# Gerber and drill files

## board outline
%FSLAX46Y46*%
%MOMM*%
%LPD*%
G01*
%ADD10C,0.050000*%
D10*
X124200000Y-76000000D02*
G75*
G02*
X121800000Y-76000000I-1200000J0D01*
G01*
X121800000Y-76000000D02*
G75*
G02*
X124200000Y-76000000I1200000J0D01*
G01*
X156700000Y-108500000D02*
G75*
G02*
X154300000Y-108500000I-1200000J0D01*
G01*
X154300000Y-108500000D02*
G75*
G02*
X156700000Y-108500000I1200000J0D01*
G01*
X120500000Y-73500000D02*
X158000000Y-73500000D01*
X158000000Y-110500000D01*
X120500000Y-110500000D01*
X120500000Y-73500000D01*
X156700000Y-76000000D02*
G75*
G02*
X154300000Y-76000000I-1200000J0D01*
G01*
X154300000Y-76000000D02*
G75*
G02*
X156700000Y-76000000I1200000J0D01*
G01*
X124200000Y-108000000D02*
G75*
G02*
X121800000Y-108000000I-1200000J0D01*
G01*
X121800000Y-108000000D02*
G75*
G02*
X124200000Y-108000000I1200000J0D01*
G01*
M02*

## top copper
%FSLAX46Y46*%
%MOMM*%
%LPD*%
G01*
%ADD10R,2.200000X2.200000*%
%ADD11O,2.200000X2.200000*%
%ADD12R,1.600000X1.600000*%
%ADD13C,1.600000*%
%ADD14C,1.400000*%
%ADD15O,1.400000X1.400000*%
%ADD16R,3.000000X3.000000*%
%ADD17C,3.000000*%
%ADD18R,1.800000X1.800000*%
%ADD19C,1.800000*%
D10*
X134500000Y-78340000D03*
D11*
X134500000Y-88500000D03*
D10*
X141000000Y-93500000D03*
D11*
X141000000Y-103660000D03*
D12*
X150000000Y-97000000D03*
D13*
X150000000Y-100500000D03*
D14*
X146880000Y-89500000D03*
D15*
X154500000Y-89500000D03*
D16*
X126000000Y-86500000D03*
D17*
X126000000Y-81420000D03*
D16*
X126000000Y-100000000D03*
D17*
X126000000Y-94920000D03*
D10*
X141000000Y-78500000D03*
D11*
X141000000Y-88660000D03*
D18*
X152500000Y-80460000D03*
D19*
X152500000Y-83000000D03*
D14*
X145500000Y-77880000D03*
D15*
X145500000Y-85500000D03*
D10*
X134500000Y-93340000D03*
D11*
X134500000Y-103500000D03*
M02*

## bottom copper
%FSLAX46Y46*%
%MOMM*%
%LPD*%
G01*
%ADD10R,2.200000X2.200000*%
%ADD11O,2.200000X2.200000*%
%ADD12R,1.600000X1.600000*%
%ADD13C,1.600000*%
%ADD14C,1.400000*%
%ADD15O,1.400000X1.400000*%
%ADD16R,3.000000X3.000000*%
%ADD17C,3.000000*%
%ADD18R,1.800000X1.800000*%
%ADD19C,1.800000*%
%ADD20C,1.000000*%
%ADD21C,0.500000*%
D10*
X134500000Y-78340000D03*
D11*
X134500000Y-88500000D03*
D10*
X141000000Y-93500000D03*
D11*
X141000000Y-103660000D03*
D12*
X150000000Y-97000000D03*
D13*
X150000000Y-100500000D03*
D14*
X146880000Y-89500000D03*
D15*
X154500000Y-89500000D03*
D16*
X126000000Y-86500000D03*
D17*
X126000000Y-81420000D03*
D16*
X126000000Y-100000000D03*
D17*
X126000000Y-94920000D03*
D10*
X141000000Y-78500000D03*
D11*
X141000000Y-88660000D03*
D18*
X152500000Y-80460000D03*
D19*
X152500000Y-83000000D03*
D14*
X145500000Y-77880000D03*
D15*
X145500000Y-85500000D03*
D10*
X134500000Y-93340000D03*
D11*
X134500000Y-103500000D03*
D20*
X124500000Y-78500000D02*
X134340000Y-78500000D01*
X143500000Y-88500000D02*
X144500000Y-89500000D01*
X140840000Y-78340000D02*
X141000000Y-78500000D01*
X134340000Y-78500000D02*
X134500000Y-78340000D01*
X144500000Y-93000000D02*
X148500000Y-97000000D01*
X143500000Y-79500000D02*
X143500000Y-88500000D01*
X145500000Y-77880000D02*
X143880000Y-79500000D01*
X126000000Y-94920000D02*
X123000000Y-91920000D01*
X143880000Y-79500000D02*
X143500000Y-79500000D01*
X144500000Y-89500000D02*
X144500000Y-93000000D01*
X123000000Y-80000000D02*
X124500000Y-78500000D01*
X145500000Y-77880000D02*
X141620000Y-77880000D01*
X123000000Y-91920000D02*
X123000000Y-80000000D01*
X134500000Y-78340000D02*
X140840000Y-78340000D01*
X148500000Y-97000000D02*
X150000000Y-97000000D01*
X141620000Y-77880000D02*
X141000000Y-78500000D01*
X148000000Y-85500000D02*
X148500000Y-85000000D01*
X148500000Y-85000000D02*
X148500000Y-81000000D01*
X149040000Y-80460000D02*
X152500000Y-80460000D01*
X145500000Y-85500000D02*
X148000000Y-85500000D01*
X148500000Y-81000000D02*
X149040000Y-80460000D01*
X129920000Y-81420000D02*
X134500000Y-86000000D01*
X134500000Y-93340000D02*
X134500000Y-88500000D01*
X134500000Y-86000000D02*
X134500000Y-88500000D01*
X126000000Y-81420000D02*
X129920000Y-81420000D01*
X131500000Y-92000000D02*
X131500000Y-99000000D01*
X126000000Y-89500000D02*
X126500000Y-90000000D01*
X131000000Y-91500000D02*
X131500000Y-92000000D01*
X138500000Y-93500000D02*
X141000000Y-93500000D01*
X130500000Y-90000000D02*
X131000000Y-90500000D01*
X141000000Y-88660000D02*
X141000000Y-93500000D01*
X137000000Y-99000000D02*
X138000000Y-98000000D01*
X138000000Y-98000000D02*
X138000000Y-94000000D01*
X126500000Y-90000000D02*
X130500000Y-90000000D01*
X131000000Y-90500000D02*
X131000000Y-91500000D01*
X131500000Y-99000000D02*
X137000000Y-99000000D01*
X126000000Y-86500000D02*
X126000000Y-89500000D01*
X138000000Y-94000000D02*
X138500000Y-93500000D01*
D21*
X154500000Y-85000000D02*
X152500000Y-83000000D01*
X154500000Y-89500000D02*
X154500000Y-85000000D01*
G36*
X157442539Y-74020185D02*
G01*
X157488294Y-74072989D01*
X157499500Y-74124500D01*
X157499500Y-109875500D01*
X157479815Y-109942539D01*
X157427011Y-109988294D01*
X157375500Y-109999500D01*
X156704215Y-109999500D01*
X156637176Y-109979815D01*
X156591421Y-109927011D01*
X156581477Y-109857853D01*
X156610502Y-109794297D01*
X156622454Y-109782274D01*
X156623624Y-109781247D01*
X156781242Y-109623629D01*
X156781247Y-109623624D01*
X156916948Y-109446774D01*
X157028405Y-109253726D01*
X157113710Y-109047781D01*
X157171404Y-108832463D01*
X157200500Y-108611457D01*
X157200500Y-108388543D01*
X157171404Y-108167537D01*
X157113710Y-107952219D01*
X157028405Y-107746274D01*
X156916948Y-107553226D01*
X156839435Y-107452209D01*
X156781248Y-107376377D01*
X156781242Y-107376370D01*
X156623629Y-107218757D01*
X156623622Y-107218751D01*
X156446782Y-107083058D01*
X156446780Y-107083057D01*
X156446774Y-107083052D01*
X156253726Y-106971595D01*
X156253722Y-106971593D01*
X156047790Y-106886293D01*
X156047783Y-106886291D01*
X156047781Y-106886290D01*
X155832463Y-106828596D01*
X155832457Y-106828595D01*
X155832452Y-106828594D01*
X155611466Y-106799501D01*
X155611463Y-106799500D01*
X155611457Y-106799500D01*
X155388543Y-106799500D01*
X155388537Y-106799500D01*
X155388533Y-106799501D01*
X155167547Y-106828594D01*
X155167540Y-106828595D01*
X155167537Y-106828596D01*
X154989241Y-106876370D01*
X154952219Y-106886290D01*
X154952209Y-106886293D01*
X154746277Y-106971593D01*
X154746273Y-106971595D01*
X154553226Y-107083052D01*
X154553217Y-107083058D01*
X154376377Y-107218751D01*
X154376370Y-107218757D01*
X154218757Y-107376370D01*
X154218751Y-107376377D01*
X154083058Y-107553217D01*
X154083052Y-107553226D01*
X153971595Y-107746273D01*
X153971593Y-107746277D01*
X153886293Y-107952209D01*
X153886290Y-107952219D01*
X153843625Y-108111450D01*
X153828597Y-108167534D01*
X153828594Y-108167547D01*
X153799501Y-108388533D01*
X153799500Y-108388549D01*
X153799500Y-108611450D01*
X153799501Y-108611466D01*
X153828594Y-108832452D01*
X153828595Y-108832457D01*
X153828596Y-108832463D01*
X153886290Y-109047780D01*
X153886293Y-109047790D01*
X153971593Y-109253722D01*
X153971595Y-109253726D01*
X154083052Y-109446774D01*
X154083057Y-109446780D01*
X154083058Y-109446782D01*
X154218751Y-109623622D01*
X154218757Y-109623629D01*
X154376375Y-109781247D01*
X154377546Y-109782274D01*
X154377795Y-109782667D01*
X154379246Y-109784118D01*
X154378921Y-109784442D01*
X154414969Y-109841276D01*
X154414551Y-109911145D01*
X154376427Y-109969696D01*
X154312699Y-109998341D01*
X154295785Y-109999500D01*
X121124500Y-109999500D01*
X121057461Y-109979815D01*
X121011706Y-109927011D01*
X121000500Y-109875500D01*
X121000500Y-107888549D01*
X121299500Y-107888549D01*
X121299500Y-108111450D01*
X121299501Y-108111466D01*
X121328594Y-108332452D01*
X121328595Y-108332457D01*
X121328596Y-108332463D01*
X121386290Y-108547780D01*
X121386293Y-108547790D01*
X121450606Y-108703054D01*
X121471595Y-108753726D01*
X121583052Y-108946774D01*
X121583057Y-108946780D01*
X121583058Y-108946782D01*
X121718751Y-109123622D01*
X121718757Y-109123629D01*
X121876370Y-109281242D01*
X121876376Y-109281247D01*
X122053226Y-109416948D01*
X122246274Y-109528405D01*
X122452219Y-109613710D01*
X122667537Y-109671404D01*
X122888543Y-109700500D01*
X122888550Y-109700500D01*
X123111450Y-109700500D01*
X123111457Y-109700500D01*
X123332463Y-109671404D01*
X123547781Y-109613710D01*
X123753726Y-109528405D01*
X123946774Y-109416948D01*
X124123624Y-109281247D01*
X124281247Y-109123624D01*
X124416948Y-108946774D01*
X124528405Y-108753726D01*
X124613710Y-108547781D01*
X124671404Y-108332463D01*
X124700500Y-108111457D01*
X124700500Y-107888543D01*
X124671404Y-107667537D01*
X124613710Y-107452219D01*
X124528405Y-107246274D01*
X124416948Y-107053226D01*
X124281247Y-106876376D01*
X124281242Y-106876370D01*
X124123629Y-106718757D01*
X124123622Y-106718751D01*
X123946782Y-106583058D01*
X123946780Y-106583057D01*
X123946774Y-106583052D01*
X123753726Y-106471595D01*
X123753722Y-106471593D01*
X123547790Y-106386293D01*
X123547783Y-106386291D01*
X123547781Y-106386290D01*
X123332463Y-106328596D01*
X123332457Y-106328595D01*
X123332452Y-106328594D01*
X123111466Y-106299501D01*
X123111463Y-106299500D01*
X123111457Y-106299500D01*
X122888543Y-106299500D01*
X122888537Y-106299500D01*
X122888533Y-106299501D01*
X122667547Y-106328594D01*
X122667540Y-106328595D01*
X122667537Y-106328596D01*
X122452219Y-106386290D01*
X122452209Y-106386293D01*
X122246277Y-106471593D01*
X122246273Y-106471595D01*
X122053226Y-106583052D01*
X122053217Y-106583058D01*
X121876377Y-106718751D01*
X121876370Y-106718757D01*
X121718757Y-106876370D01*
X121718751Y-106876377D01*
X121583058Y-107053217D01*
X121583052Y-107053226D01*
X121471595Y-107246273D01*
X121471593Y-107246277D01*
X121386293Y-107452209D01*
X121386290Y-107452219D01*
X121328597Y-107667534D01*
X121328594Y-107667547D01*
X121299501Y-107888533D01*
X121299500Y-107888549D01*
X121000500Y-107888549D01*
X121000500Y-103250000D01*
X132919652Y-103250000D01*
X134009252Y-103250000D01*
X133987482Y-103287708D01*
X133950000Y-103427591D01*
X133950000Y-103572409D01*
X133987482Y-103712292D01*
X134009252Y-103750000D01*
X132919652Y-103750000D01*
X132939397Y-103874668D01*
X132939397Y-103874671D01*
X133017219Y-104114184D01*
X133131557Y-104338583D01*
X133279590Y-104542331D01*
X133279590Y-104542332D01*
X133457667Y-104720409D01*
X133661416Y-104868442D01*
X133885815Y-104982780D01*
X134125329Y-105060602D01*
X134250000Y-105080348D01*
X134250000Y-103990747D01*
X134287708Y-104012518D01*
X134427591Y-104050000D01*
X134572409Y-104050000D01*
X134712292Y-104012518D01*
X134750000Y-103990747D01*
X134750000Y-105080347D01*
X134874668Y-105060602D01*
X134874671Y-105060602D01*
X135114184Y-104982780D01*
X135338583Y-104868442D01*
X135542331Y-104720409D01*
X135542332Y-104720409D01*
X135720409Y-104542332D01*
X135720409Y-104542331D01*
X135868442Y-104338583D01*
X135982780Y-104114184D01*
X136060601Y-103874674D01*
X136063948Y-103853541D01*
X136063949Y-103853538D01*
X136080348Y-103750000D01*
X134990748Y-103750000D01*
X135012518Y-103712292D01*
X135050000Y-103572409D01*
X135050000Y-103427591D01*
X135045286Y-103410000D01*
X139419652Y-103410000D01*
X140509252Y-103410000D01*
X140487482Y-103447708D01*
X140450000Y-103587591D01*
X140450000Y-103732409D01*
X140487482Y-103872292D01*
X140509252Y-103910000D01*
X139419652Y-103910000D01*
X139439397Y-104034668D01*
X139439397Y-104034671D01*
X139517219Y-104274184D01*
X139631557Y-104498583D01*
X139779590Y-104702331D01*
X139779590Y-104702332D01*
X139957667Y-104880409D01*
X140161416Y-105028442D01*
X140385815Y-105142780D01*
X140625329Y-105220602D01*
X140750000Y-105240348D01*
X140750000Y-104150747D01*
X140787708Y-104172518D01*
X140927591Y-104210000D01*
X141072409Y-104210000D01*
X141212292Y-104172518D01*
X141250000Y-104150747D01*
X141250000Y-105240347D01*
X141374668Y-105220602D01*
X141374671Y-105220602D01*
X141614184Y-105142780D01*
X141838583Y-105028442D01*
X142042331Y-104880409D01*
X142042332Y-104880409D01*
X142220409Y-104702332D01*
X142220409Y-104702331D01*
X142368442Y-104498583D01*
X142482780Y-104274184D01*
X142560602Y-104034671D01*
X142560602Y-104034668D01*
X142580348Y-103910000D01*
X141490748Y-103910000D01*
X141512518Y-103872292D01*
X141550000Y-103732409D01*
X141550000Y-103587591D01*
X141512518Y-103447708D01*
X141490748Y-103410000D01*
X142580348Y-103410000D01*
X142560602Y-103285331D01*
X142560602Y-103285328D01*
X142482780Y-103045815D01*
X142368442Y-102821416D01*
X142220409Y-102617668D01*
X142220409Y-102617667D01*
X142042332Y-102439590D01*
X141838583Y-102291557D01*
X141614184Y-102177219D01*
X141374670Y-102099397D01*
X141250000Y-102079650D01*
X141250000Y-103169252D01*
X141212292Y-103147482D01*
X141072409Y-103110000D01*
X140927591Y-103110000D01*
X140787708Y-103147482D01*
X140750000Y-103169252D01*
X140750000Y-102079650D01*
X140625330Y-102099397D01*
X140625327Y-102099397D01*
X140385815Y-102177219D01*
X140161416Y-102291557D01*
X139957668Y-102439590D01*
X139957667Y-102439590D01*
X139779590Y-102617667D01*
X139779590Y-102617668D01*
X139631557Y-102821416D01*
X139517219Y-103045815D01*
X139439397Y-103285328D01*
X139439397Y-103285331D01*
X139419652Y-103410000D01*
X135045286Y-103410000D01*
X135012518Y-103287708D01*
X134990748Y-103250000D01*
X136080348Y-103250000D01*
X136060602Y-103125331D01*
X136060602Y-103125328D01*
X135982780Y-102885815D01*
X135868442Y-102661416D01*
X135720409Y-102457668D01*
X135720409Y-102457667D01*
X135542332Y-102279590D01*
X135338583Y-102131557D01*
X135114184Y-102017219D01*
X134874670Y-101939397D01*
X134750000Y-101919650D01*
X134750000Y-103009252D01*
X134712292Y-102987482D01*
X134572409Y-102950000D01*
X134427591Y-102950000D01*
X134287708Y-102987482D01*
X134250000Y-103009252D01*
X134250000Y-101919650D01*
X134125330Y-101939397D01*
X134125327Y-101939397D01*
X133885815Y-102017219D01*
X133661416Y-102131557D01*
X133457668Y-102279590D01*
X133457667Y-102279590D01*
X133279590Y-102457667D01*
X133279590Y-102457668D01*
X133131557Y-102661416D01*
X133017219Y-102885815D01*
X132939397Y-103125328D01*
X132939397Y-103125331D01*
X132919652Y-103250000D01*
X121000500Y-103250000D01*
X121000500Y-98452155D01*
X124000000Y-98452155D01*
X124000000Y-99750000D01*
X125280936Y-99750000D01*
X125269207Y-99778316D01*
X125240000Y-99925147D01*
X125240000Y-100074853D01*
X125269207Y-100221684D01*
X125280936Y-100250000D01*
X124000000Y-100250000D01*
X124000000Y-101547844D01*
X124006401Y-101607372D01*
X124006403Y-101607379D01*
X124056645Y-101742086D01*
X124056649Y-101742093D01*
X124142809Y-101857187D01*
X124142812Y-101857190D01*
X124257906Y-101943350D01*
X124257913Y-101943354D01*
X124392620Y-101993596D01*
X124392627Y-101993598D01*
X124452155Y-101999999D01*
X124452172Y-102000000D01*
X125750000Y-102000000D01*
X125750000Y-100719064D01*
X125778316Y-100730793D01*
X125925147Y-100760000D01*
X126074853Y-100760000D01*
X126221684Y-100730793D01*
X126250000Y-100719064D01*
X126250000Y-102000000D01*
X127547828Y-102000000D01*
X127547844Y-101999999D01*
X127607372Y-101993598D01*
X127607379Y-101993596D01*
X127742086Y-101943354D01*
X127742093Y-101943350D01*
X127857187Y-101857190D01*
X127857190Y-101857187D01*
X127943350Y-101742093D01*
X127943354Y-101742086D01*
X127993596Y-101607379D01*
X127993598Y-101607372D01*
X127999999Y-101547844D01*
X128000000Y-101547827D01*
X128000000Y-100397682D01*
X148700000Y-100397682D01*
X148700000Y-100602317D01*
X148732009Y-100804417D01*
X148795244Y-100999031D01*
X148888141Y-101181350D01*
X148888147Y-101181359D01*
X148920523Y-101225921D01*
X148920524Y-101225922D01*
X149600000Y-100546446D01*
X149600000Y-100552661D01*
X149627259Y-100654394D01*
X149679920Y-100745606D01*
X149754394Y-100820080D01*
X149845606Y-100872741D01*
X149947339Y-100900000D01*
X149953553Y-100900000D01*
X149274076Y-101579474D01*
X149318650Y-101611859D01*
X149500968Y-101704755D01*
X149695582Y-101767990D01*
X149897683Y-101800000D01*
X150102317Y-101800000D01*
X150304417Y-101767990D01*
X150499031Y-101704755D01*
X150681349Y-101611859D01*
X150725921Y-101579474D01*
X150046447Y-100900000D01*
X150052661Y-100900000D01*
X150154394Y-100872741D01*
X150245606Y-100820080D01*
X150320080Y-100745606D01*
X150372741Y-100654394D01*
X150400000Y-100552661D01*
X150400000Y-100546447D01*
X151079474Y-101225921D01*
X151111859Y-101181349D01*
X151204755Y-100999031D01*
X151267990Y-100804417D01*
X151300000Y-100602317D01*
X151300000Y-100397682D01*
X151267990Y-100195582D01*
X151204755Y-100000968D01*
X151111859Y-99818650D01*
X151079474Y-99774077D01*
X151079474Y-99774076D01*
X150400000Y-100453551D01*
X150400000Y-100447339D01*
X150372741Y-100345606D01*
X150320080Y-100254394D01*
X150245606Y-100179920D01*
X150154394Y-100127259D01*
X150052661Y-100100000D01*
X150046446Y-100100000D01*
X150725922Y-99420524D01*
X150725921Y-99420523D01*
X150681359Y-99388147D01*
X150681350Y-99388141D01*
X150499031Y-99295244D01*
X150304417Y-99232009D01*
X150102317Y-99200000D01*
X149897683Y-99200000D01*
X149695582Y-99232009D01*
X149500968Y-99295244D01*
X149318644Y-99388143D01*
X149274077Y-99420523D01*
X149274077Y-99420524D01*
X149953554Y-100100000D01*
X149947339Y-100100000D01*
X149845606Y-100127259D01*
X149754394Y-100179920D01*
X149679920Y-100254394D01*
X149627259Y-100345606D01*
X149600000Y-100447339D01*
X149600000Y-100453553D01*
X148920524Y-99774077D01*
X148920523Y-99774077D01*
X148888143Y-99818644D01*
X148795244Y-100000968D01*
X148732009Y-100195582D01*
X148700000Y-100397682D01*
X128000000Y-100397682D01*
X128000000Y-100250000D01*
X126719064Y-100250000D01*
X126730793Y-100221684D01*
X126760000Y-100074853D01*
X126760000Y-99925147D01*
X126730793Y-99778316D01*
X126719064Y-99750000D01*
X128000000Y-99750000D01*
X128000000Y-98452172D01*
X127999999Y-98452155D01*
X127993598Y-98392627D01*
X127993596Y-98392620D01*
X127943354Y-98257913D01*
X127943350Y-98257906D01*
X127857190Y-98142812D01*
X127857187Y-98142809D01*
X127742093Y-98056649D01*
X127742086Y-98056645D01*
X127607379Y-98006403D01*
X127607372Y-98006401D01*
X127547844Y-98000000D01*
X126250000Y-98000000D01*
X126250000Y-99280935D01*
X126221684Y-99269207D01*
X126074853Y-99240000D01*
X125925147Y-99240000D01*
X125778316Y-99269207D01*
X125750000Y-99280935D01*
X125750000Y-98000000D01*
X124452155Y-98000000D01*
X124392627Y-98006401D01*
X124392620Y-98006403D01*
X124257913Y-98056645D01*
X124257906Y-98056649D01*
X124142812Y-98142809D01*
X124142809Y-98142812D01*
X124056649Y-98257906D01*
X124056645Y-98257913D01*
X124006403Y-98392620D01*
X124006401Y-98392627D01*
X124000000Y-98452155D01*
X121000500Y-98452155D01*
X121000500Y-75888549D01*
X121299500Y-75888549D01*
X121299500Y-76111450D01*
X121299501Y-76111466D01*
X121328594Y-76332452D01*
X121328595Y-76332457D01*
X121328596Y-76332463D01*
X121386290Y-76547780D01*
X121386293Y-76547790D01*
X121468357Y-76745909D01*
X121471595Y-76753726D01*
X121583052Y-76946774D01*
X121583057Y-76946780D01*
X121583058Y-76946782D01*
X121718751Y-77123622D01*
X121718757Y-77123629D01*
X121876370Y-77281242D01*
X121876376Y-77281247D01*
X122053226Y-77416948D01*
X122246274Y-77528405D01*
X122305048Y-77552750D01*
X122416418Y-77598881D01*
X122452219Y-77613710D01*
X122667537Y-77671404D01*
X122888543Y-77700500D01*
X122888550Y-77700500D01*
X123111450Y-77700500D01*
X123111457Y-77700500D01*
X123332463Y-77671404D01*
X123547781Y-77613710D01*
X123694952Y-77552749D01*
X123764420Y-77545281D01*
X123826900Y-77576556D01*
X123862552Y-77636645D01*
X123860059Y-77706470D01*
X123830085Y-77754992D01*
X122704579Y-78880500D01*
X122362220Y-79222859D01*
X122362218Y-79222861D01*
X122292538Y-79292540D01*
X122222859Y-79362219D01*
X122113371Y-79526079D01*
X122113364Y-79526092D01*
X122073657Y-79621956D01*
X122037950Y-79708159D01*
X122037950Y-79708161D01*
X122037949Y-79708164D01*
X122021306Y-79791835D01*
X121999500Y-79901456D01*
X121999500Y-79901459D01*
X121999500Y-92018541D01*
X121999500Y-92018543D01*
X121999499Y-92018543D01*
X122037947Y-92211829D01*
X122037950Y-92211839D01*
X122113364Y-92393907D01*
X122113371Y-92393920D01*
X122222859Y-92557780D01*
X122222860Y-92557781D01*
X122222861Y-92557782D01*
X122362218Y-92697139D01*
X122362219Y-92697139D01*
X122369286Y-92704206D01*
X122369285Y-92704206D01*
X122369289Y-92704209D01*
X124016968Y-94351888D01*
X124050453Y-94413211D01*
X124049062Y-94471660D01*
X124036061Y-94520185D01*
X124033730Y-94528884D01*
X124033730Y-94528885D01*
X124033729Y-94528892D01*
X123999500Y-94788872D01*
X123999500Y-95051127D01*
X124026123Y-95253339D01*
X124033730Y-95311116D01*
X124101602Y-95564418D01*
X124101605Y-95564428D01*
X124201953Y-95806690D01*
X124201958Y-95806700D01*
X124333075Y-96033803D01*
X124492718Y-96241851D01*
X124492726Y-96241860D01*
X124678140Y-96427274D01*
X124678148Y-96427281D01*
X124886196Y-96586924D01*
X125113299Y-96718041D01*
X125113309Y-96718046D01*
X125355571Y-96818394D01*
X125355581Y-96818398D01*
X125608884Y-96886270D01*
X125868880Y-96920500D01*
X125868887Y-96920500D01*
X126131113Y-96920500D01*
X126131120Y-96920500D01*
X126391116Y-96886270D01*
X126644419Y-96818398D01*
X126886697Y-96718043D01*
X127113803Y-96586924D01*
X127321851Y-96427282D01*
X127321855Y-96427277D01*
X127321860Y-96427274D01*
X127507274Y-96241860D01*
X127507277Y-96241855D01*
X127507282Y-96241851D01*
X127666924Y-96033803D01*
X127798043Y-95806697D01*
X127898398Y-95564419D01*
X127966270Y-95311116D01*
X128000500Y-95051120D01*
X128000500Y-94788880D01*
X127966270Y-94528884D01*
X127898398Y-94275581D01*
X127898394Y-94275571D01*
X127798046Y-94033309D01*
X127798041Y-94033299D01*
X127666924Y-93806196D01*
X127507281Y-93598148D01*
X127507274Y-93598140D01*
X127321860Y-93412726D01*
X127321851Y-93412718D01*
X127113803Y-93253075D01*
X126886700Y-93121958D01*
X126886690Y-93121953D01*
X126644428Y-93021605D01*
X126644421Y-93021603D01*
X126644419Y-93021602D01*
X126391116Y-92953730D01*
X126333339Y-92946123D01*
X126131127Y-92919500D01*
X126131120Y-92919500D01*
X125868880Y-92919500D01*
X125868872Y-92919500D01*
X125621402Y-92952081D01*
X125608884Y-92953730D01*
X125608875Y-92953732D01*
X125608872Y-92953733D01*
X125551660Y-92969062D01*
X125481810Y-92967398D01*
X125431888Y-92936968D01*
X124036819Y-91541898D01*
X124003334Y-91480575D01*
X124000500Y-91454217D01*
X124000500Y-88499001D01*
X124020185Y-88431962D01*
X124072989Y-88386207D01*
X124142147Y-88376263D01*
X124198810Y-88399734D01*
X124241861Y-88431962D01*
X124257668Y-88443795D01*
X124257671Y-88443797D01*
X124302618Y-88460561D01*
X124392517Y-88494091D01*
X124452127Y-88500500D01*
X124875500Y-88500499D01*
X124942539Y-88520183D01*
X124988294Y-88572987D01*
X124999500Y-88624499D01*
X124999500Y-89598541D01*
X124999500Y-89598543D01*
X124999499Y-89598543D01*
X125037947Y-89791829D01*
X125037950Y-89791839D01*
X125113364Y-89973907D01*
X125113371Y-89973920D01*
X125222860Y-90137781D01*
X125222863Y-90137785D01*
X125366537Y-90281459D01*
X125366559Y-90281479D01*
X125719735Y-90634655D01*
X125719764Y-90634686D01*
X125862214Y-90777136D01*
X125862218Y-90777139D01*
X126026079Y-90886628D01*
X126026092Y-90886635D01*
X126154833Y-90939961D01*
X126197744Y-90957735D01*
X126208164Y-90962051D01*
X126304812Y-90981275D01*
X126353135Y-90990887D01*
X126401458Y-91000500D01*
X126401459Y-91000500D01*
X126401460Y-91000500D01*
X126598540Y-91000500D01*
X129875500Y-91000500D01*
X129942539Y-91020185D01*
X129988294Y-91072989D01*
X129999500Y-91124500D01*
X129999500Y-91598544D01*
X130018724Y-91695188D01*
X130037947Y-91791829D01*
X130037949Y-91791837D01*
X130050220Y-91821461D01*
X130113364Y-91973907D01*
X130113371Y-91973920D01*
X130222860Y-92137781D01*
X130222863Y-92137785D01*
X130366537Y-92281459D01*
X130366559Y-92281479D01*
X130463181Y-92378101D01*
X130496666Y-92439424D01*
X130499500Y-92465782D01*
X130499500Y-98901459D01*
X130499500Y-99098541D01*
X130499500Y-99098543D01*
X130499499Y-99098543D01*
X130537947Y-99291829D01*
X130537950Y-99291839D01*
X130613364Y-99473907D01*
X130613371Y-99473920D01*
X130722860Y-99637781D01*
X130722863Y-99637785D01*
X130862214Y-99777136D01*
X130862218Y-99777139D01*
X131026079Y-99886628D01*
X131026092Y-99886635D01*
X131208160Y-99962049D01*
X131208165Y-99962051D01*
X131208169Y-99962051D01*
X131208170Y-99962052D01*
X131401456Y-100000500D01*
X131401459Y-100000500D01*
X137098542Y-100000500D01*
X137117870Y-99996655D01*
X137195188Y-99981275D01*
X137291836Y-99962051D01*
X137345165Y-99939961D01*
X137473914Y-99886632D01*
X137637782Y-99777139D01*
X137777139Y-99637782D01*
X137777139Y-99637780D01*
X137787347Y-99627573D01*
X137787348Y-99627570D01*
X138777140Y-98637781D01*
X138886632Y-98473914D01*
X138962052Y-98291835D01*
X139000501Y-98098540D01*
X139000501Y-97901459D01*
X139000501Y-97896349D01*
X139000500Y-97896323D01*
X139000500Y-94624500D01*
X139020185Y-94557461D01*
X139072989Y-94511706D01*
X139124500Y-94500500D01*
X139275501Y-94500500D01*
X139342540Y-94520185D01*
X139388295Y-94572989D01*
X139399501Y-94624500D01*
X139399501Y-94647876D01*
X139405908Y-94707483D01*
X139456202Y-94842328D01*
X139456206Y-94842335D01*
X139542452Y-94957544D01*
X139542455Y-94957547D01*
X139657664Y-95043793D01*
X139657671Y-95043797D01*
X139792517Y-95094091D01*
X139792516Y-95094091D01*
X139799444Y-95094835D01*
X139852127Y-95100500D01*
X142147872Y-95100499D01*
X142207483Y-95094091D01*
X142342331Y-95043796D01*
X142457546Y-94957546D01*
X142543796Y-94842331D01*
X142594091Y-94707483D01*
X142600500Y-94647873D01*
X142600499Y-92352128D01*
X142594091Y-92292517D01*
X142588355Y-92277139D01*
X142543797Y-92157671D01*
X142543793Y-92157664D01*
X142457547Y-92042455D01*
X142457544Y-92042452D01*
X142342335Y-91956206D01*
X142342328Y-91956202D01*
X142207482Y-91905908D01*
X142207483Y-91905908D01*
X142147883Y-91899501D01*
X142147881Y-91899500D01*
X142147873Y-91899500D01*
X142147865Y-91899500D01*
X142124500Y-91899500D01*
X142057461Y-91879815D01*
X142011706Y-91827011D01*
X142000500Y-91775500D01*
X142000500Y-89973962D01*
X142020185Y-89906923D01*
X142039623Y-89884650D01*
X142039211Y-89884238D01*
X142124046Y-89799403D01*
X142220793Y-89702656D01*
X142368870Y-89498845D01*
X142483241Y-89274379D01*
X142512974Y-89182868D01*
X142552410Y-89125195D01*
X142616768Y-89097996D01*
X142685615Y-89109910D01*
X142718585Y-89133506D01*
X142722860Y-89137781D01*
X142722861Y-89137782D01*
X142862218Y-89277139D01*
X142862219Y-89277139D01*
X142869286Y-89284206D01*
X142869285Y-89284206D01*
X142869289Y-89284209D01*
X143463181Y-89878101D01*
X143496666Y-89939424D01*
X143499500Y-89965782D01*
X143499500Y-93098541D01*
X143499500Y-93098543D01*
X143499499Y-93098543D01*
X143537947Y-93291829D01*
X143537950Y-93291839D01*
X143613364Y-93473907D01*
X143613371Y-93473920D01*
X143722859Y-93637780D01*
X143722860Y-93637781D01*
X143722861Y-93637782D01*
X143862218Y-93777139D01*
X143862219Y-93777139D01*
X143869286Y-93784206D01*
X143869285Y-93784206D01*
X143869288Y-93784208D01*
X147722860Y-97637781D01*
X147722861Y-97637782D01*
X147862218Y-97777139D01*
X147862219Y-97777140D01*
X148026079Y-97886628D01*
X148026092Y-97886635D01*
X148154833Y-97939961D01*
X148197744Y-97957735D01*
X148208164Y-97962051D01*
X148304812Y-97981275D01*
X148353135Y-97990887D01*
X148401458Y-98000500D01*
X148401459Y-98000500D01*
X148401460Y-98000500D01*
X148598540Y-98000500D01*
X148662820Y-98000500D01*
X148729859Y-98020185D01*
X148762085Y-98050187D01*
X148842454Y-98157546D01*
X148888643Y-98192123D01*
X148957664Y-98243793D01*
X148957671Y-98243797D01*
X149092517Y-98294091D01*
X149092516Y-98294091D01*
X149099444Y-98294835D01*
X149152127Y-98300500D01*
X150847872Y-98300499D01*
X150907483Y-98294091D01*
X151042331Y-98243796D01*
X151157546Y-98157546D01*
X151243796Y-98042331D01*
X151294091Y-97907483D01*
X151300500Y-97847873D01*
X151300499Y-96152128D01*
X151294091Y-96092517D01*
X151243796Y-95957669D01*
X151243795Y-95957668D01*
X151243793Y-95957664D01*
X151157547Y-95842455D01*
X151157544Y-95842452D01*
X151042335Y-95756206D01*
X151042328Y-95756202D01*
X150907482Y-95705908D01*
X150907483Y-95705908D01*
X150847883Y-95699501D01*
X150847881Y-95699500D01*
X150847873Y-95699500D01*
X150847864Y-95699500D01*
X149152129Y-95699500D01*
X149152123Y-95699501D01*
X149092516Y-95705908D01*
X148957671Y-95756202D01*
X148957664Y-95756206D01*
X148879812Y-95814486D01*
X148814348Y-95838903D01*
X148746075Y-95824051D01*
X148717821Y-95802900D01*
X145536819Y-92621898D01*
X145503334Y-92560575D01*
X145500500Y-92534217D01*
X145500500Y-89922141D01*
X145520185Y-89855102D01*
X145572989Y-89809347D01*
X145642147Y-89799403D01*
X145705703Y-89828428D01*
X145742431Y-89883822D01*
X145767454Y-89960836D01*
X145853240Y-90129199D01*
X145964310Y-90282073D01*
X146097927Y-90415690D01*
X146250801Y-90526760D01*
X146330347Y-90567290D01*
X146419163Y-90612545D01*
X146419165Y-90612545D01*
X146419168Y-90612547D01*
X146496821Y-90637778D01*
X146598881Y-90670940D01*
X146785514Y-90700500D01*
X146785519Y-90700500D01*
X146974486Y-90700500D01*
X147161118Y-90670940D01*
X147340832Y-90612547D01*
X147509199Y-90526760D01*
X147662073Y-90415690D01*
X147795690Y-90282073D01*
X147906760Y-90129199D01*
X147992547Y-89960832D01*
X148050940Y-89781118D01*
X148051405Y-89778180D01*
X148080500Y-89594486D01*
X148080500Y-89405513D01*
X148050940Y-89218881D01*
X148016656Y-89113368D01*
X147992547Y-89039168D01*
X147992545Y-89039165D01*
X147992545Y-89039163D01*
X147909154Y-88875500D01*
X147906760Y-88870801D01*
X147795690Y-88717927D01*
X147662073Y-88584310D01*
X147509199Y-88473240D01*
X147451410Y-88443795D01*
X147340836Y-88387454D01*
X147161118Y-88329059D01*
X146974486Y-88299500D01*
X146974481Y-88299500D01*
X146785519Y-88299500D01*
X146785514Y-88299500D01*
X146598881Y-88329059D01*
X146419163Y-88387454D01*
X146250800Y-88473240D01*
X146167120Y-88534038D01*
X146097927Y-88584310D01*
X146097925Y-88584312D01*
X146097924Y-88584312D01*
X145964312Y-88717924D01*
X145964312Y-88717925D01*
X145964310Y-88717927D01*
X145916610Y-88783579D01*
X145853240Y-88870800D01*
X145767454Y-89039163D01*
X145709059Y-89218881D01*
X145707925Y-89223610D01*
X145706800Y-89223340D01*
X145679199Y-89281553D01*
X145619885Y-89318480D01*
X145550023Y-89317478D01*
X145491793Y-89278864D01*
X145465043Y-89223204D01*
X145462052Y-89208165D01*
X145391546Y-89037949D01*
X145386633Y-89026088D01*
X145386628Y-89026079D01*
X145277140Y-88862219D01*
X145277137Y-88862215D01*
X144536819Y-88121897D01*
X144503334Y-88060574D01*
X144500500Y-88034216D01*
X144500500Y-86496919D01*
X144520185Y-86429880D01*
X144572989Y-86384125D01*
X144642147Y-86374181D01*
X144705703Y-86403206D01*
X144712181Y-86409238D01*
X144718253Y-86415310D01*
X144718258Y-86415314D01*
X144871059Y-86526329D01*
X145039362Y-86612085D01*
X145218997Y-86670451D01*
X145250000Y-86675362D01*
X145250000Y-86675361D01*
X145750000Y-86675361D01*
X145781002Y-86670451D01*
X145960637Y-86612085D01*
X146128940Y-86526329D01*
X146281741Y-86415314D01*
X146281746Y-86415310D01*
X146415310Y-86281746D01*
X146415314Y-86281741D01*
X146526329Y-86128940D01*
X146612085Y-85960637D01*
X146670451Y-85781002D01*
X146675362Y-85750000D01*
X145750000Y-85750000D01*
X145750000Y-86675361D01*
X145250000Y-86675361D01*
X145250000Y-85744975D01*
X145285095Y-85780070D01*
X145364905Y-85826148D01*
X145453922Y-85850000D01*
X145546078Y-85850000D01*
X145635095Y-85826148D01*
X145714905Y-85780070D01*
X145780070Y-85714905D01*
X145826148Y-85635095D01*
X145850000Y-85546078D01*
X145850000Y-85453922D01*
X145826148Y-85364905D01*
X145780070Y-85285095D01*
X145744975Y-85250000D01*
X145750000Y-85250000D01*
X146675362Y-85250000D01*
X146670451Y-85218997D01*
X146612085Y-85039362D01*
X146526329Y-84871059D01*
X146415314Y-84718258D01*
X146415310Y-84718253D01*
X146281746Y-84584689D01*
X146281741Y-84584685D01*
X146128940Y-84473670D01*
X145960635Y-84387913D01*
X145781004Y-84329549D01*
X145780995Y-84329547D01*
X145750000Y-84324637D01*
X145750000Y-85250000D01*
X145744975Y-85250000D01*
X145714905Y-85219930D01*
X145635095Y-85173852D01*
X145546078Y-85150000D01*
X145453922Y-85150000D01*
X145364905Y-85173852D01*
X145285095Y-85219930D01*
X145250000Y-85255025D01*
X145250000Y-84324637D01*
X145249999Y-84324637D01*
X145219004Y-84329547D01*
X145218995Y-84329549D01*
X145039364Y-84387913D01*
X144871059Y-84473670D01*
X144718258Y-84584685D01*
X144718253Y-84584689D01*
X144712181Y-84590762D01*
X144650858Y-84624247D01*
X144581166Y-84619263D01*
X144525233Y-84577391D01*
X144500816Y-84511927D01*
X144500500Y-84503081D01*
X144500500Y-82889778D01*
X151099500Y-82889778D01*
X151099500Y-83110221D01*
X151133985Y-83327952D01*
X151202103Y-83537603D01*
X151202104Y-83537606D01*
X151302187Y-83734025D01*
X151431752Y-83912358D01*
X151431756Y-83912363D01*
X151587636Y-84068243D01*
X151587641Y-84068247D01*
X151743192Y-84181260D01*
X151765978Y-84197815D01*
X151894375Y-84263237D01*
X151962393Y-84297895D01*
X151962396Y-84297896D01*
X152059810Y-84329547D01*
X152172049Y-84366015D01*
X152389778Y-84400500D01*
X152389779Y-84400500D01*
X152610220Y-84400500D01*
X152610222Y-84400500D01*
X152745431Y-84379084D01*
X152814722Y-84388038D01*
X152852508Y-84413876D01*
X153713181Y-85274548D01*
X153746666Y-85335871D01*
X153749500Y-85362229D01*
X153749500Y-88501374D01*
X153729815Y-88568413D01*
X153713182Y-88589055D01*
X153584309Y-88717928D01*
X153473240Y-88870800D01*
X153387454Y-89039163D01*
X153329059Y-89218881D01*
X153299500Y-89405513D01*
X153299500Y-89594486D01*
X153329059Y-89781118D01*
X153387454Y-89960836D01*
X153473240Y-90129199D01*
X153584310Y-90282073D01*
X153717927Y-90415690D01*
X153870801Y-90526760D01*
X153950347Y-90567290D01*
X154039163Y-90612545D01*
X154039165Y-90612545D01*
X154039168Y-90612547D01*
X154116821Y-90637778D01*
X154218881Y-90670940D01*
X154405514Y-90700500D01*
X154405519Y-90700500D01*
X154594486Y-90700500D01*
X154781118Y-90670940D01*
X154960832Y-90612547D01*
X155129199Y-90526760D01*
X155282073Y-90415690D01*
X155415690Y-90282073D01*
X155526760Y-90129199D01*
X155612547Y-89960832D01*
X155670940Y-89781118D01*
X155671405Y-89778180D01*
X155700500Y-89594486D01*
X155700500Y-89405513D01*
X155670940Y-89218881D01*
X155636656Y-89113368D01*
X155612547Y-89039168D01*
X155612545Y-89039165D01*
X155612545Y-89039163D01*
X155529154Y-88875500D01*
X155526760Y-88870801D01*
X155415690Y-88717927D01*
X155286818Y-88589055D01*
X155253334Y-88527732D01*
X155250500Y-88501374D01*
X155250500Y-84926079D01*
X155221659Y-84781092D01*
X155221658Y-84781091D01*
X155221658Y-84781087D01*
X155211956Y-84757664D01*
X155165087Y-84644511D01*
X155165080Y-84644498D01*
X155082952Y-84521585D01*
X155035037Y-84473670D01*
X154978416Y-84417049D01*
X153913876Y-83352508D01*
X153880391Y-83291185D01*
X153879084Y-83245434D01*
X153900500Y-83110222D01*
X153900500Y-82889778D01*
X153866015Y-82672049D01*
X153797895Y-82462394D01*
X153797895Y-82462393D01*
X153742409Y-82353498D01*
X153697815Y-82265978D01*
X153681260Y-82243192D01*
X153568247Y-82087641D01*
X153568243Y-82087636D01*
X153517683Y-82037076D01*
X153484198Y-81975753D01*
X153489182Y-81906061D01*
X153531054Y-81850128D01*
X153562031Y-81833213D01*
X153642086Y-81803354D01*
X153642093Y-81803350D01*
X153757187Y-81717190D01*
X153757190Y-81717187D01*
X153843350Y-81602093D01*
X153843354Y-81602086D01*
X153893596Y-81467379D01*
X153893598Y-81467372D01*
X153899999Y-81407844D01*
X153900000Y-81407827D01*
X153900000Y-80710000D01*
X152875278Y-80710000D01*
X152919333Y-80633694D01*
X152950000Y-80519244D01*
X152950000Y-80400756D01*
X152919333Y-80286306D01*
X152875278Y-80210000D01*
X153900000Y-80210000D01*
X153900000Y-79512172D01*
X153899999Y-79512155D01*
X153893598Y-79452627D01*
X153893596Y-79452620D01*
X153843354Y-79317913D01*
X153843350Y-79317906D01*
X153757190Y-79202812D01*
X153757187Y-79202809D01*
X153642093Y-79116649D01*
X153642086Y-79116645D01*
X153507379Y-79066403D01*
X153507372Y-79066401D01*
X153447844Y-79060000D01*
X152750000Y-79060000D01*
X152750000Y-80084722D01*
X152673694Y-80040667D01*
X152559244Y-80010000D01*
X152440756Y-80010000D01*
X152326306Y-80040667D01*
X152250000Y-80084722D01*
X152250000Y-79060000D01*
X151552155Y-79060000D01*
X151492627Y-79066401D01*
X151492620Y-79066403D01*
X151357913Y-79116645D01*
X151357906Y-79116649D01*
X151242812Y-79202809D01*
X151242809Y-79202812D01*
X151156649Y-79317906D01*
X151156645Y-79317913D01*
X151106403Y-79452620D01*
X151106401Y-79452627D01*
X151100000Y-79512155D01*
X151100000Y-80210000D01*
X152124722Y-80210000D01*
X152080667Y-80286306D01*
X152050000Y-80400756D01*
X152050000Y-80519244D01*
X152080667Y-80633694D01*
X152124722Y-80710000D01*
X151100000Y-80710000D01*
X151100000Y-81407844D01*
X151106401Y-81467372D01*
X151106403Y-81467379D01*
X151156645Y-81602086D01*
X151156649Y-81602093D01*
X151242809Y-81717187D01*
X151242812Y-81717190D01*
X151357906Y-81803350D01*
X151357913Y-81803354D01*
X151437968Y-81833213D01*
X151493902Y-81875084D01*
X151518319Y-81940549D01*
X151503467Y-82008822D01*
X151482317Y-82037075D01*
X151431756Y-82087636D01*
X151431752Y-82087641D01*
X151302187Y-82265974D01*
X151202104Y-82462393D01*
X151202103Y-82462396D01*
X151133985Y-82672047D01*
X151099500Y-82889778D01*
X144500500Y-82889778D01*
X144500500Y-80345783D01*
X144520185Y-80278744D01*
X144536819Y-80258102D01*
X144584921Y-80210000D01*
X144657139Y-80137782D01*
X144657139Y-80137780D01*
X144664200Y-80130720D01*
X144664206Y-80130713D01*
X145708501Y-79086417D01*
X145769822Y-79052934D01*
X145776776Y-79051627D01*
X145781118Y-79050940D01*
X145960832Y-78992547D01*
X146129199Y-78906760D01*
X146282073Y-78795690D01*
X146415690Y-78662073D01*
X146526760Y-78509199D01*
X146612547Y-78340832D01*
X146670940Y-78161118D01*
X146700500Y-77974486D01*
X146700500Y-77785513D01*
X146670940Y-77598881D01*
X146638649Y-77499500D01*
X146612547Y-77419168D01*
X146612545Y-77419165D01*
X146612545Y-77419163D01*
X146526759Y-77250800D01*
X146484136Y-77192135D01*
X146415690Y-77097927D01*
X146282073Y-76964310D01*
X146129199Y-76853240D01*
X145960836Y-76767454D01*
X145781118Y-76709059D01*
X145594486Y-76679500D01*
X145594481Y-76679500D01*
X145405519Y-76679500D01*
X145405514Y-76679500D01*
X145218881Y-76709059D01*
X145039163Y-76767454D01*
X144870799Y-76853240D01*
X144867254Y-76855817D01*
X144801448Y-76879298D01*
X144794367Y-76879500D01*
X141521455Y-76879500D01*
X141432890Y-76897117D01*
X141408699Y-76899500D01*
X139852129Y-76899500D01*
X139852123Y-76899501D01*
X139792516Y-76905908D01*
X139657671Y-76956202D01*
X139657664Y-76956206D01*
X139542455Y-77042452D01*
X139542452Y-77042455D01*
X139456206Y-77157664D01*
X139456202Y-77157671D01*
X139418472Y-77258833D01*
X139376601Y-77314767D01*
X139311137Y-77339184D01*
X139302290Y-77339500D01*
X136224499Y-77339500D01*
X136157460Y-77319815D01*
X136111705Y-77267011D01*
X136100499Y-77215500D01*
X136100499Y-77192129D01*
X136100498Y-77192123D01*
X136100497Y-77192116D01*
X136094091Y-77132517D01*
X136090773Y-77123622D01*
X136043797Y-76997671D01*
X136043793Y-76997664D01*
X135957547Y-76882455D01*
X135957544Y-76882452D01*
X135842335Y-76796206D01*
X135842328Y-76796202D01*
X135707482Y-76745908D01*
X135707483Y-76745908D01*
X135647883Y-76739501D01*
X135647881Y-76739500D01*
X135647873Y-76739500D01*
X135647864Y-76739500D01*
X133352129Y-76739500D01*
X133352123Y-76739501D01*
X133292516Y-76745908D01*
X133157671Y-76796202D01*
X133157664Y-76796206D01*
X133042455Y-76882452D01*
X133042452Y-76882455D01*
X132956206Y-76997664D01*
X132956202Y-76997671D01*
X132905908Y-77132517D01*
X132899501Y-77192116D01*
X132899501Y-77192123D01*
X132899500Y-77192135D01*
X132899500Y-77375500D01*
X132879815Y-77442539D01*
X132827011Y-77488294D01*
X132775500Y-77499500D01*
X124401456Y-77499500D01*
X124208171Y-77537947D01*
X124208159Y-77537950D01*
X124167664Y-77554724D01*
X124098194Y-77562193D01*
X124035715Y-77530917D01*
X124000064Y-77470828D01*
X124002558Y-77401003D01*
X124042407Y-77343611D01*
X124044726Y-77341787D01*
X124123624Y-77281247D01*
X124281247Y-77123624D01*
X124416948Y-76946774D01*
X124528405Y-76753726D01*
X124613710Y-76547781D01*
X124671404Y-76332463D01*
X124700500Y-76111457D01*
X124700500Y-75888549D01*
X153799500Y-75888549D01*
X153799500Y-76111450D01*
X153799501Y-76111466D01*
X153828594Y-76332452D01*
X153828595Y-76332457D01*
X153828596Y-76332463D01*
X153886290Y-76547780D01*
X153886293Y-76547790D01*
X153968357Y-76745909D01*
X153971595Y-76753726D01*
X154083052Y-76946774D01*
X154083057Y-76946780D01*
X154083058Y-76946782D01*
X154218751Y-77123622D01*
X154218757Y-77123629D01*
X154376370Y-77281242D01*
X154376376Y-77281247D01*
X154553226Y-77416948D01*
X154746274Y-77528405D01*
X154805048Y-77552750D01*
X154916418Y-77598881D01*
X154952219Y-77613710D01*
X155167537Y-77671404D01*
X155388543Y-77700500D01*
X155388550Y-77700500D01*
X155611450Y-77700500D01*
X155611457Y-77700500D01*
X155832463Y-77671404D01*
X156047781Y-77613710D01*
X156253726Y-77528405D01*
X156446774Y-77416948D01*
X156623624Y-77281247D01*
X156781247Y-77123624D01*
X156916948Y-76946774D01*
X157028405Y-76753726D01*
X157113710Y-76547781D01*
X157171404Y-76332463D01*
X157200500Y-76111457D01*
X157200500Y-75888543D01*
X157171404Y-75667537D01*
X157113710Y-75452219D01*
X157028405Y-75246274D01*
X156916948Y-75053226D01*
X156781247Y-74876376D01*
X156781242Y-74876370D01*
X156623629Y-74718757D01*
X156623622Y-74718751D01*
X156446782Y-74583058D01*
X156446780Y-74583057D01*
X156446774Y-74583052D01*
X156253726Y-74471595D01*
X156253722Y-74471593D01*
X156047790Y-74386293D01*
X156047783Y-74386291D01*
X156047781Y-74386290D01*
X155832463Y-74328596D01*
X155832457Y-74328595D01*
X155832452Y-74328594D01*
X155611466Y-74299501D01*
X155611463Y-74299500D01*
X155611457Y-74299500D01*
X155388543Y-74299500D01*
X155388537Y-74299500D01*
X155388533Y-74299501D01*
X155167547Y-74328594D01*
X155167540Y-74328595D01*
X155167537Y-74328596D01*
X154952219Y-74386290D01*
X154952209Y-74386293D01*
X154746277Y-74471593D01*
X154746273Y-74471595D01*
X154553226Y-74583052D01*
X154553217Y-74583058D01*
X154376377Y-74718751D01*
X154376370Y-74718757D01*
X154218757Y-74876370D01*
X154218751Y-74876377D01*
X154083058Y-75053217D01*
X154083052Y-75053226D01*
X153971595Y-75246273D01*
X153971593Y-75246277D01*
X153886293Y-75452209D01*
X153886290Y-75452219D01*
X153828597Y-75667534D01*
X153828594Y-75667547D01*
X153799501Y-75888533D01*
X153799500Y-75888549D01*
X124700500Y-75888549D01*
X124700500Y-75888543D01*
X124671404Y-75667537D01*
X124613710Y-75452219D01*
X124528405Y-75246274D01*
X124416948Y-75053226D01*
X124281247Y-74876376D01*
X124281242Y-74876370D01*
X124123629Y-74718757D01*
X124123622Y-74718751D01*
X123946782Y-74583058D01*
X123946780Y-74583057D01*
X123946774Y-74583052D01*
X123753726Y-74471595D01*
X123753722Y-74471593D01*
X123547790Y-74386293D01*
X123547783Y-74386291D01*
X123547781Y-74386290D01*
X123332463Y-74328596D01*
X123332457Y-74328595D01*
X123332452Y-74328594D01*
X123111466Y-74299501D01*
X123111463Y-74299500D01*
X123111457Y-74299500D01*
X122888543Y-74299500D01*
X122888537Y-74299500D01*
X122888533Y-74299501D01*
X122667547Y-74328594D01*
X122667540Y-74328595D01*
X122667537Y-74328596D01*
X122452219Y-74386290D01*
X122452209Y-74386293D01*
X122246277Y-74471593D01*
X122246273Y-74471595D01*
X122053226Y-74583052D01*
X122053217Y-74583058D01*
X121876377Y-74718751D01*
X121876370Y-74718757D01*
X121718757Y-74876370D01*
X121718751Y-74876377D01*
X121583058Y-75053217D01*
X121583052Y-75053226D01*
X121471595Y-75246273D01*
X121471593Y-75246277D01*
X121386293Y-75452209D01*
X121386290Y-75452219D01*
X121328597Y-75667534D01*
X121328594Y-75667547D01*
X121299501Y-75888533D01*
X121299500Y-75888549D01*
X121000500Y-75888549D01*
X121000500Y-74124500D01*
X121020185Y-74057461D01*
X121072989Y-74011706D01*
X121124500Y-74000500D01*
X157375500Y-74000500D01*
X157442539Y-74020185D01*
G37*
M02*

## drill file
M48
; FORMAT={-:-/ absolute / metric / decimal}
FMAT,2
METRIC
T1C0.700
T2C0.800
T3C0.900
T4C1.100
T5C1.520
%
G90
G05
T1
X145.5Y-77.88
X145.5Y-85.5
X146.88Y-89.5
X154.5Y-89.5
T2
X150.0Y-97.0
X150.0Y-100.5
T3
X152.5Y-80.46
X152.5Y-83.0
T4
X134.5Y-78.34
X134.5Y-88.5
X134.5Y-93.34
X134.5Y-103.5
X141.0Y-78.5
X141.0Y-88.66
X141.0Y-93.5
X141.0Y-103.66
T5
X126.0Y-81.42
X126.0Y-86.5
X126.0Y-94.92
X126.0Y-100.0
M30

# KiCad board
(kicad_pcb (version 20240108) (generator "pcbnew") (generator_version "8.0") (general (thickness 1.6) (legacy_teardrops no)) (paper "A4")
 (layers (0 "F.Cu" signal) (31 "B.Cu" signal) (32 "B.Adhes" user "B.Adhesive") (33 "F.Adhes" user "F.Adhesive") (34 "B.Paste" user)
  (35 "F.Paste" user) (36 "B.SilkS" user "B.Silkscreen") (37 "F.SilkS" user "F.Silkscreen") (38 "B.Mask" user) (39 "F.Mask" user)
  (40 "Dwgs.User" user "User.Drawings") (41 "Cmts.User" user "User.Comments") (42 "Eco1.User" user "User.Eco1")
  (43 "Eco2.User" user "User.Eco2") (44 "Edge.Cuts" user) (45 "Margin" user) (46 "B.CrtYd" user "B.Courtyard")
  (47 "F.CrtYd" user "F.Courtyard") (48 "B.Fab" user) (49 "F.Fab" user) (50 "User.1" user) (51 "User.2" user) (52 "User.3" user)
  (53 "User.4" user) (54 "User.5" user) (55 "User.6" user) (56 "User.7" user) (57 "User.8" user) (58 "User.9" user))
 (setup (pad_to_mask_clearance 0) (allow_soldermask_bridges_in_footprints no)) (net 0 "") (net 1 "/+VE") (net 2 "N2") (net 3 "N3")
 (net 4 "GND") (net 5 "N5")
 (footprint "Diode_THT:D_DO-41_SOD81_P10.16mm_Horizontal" (layer "F.Cu") (at 134.5 78.34 -90)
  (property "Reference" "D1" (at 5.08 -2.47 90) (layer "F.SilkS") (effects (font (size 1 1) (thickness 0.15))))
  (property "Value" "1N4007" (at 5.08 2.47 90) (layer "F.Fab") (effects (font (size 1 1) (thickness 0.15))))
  (pad "1" thru_hole rect (at 0 0 270) (size 2.2 2.2) (drill 1.1) (layers "*.Cu" "*.Mask") (remove_unused_layers no) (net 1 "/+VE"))
  (pad "2" thru_hole oval (at 10.16 0 270) (size 2.2 2.2) (drill 1.1) (layers "*.Cu" "*.Mask") (remove_unused_layers no) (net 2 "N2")))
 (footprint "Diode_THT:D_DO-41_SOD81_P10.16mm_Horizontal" (layer "F.Cu") (at 141 93.5 -90)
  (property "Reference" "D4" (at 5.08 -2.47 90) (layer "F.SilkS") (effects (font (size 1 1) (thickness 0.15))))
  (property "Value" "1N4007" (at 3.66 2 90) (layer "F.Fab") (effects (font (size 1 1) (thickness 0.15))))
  (pad "1" thru_hole rect (at 0 0 270) (size 2.2 2.2) (drill 1.1) (layers "*.Cu" "*.Mask") (remove_unused_layers no) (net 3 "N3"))
  (pad "2" thru_hole oval (at 10.16 0 270) (size 2.2 2.2) (drill 1.1) (layers "*.Cu" "*.Mask") (remove_unused_layers no) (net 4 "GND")))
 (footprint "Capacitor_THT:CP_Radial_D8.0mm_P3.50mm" (layer "F.Cu") (at 150 97 -90)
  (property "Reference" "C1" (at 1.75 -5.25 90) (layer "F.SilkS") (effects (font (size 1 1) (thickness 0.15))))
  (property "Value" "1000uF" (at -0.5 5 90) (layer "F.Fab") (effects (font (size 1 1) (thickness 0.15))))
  (pad "1" thru_hole rect (at 0 0 270) (size 1.6 1.6) (drill 0.8) (layers "*.Cu" "*.Mask") (remove_unused_layers no) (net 1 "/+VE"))
  (pad "2" thru_hole circle (at 3.5 0 270) (size 1.6 1.6) (drill 0.8) (layers "*.Cu" "*.Mask") (remove_unused_layers no) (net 4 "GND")))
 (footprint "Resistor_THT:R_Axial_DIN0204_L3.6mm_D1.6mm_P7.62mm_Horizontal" (layer "F.Cu") (at 146.88 89.5)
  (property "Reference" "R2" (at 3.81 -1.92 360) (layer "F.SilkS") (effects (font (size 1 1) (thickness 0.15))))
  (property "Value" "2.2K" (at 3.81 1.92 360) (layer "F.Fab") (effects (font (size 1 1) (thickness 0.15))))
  (pad "1" thru_hole circle (at 0 0) (size 1.4 1.4) (drill 0.7) (layers "*.Cu" "*.Mask") (remove_unused_layers no) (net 1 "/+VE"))
  (pad "2" thru_hole oval (at 7.62 0) (size 1.4 1.4) (drill 0.7) (layers "*.Cu" "*.Mask") (remove_unused_layers no) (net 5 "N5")))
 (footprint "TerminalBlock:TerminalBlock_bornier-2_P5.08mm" (layer "F.Cu") (at 126 86.5 90)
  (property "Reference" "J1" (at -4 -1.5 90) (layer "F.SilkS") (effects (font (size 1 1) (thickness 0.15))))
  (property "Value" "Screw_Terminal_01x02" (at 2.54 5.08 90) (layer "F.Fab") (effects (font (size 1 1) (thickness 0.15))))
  (pad "1" thru_hole rect (at 0 0 90) (size 3 3) (drill 1.52) (layers "*.Cu" "*.Mask") (remove_unused_layers no) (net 3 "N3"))
  (pad "2" thru_hole circle (at 5.08 0 90) (size 3 3) (drill 1.52) (layers "*.Cu" "*.Mask") (remove_unused_layers no) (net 2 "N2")))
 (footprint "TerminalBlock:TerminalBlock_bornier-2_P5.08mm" (layer "F.Cu") (at 126 100 90)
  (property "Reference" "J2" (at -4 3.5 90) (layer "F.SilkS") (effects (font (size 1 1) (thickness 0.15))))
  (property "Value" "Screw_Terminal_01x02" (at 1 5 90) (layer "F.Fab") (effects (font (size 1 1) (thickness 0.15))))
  (pad "1" thru_hole rect (at 0 0 90) (size 3 3) (drill 1.52) (layers "*.Cu" "*.Mask") (remove_unused_layers no) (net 4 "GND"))
  (pad "2" thru_hole circle (at 5.08 0 90) (size 3 3) (drill 1.52) (layers "*.Cu" "*.Mask") (remove_unused_layers no) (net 1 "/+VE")))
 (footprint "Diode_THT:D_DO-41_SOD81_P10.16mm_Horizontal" (layer "F.Cu") (at 141 78.5 -90)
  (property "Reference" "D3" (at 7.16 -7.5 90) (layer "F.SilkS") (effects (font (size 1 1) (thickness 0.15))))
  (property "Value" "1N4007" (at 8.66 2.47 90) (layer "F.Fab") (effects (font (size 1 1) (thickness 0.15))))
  (pad "1" thru_hole rect (at 0 0 270) (size 2.2 2.2) (drill 1.1) (layers "*.Cu" "*.Mask") (remove_unused_layers no) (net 1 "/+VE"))
  (pad "2" thru_hole oval (at 10.16 0 270) (size 2.2 2.2) (drill 1.1) (layers "*.Cu" "*.Mask") (remove_unused_layers no) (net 3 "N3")))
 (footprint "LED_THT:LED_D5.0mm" (layer "F.Cu") (at 152.5 80.46 -90)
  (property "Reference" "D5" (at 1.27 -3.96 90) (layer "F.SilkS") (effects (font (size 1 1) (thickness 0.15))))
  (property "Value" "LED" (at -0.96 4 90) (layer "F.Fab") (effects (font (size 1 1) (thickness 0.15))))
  (pad "1" thru_hole rect (at 0 0 270) (size 1.8 1.8) (drill 0.9) (layers "*.Cu" "*.Mask") (remove_unused_layers no) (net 4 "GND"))
  (pad "2" thru_hole circle (at 2.54 0 270) (size 1.8 1.8) (drill 0.9) (layers "*.Cu" "*.Mask") (remove_unused_layers no) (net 5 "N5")))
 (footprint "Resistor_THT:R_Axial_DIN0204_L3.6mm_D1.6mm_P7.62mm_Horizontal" (layer "F.Cu") (at 145.5 77.88 -90)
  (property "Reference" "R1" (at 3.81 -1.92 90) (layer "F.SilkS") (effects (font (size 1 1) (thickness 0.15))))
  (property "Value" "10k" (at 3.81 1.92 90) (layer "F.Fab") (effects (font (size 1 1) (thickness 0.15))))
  (pad "1" thru_hole circle (at 0 0 270) (size 1.4 1.4) (drill 0.7) (layers "*.Cu" "*.Mask") (remove_unused_layers no) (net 1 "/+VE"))
  (pad "2" thru_hole oval (at 7.62 0 270) (size 1.4 1.4) (drill 0.7) (layers "*.Cu" "*.Mask") (remove_unused_layers no) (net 4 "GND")))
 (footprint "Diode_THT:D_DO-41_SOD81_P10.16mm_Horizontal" (layer "F.Cu") (at 134.5 93.34 -90)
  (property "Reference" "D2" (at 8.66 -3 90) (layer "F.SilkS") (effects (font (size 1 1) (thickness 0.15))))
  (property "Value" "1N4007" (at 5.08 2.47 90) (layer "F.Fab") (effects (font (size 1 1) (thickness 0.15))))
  (pad "1" thru_hole rect (at 0 0 270) (size 2.2 2.2) (drill 1.1) (layers "*.Cu" "*.Mask") (remove_unused_layers no) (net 2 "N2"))
  (pad "2" thru_hole oval (at 10.16 0 270) (size 2.2 2.2) (drill 1.1) (layers "*.Cu" "*.Mask") (remove_unused_layers no) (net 4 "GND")))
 (gr_circle (center 123 76) (end 124.2 76) (stroke (width 0.05) (type default)) (fill none) (layer "Edge.Cuts"))
 (gr_circle (center 155.5 108.5) (end 156.7 108.5) (stroke (width 0.05) (type default)) (fill none) (layer "Edge.Cuts"))
 (gr_rect (start 120.5 73.5) (end 158 110.5) (stroke (width 0.05) (type default)) (fill none) (layer "Edge.Cuts"))
 (gr_circle (center 155.5 76) (end 156.7 76) (stroke (width 0.05) (type default)) (fill none) (layer "Edge.Cuts"))
 (gr_circle (center 123 108) (end 124.2 108) (stroke (width 0.05) (type default)) (fill none) (layer "Edge.Cuts"))
 (segment (start 124.5 78.5) (end 134.34 78.5) (width 1) (layer "B.Cu") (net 1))
 (segment (start 143.5 88.5) (end 144.5 89.5) (width 1) (layer "B.Cu") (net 1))
 (segment (start 140.84 78.34) (end 141 78.5) (width 1) (layer "B.Cu") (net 1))
 (segment (start 134.34 78.5) (end 134.5 78.34) (width 1) (layer "B.Cu") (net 1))
 (segment (start 144.5 93) (end 148.5 97) (width 1) (layer "B.Cu") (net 1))
 (segment (start 143.5 79.5) (end 143.5 88.5) (width 1) (layer "B.Cu") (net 1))
 (segment (start 145.5 77.88) (end 143.88 79.5) (width 1) (layer "B.Cu") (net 1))
 (segment (start 126 94.92) (end 123 91.92) (width 1) (layer "B.Cu") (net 1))
 (segment (start 143.88 79.5) (end 143.5 79.5) (width 1) (layer "B.Cu") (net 1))
 (segment (start 144.5 89.5) (end 144.5 93) (width 1) (layer "B.Cu") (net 1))
 (segment (start 123 80) (end 124.5 78.5) (width 1) (layer "B.Cu") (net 1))
 (segment (start 145.5 77.88) (end 141.62 77.88) (width 1) (layer "B.Cu") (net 1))
 (segment (start 123 91.92) (end 123 80) (width 1) (layer "B.Cu") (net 1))
 (segment (start 134.5 78.34) (end 140.84 78.34) (width 1) (layer "B.Cu") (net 1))
 (segment (start 148.5 97) (end 150 97) (width 1) (layer "B.Cu") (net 1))
 (segment (start 141.62 77.88) (end 141 78.5) (width 1) (layer "B.Cu") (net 1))
 (segment (start 148 85.5) (end 148.5 85) (width 1) (layer "B.Cu") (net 4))
 (segment (start 148.5 85) (end 148.5 81) (width 1) (layer "B.Cu") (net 4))
 (segment (start 149.04 80.46) (end 152.5 80.46) (width 1) (layer "B.Cu") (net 4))
 (segment (start 145.5 85.5) (end 148 85.5) (width 1) (layer "B.Cu") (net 4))
 (segment (start 148.5 81) (end 149.04 80.46) (width 1) (layer "B.Cu") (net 4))
 (segment (start 129.92 81.42) (end 134.5 86) (width 1) (layer "B.Cu") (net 2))
 (segment (start 134.5 93.34) (end 134.5 88.5) (width 1) (layer "B.Cu") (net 2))
 (segment (start 134.5 86) (end 134.5 88.5) (width 1) (layer "B.Cu") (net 2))
 (segment (start 126 81.42) (end 129.92 81.42) (width 1) (layer "B.Cu") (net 2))
 (segment (start 131.5 92) (end 131.5 99) (width 1) (layer "B.Cu") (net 3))
 (segment (start 126 89.5) (end 126.5 90) (width 1) (layer "B.Cu") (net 3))
 (segment (start 131 91.5) (end 131.5 92) (width 1) (layer "B.Cu") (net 3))
 (segment (start 138.5 93.5) (end 141 93.5) (width 1) (layer "B.Cu") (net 3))
 (segment (start 130.5 90) (end 131 90.5) (width 1) (layer "B.Cu") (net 3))
 (segment (start 141 88.66) (end 141 93.5) (width 1) (layer "B.Cu") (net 3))
 (segment (start 137 99) (end 138 98) (width 1) (layer "B.Cu") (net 3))
 (segment (start 138 98) (end 138 94) (width 1) (layer "B.Cu") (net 3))
 (segment (start 126.5 90) (end 130.5 90) (width 1) (layer "B.Cu") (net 3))
 (segment (start 131 90.5) (end 131 91.5) (width 1) (layer "B.Cu") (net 3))
 (segment (start 131.5 99) (end 137 99) (width 1) (layer "B.Cu") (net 3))
 (segment (start 126 86.5) (end 126 89.5) (width 1) (layer "B.Cu") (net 3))
 (segment (start 138 94) (end 138.5 93.5) (width 1) (layer "B.Cu") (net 3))
 (segment (start 154.5 85) (end 152.5 83) (width 0.5) (layer "B.Cu") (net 5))
 (segment (start 154.5 89.5) (end 154.5 85) (width 0.5) (layer "B.Cu") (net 5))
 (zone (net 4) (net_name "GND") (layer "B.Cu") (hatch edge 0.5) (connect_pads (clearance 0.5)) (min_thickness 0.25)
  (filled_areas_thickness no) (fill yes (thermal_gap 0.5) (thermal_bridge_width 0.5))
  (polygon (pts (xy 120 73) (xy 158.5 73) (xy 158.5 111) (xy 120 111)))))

